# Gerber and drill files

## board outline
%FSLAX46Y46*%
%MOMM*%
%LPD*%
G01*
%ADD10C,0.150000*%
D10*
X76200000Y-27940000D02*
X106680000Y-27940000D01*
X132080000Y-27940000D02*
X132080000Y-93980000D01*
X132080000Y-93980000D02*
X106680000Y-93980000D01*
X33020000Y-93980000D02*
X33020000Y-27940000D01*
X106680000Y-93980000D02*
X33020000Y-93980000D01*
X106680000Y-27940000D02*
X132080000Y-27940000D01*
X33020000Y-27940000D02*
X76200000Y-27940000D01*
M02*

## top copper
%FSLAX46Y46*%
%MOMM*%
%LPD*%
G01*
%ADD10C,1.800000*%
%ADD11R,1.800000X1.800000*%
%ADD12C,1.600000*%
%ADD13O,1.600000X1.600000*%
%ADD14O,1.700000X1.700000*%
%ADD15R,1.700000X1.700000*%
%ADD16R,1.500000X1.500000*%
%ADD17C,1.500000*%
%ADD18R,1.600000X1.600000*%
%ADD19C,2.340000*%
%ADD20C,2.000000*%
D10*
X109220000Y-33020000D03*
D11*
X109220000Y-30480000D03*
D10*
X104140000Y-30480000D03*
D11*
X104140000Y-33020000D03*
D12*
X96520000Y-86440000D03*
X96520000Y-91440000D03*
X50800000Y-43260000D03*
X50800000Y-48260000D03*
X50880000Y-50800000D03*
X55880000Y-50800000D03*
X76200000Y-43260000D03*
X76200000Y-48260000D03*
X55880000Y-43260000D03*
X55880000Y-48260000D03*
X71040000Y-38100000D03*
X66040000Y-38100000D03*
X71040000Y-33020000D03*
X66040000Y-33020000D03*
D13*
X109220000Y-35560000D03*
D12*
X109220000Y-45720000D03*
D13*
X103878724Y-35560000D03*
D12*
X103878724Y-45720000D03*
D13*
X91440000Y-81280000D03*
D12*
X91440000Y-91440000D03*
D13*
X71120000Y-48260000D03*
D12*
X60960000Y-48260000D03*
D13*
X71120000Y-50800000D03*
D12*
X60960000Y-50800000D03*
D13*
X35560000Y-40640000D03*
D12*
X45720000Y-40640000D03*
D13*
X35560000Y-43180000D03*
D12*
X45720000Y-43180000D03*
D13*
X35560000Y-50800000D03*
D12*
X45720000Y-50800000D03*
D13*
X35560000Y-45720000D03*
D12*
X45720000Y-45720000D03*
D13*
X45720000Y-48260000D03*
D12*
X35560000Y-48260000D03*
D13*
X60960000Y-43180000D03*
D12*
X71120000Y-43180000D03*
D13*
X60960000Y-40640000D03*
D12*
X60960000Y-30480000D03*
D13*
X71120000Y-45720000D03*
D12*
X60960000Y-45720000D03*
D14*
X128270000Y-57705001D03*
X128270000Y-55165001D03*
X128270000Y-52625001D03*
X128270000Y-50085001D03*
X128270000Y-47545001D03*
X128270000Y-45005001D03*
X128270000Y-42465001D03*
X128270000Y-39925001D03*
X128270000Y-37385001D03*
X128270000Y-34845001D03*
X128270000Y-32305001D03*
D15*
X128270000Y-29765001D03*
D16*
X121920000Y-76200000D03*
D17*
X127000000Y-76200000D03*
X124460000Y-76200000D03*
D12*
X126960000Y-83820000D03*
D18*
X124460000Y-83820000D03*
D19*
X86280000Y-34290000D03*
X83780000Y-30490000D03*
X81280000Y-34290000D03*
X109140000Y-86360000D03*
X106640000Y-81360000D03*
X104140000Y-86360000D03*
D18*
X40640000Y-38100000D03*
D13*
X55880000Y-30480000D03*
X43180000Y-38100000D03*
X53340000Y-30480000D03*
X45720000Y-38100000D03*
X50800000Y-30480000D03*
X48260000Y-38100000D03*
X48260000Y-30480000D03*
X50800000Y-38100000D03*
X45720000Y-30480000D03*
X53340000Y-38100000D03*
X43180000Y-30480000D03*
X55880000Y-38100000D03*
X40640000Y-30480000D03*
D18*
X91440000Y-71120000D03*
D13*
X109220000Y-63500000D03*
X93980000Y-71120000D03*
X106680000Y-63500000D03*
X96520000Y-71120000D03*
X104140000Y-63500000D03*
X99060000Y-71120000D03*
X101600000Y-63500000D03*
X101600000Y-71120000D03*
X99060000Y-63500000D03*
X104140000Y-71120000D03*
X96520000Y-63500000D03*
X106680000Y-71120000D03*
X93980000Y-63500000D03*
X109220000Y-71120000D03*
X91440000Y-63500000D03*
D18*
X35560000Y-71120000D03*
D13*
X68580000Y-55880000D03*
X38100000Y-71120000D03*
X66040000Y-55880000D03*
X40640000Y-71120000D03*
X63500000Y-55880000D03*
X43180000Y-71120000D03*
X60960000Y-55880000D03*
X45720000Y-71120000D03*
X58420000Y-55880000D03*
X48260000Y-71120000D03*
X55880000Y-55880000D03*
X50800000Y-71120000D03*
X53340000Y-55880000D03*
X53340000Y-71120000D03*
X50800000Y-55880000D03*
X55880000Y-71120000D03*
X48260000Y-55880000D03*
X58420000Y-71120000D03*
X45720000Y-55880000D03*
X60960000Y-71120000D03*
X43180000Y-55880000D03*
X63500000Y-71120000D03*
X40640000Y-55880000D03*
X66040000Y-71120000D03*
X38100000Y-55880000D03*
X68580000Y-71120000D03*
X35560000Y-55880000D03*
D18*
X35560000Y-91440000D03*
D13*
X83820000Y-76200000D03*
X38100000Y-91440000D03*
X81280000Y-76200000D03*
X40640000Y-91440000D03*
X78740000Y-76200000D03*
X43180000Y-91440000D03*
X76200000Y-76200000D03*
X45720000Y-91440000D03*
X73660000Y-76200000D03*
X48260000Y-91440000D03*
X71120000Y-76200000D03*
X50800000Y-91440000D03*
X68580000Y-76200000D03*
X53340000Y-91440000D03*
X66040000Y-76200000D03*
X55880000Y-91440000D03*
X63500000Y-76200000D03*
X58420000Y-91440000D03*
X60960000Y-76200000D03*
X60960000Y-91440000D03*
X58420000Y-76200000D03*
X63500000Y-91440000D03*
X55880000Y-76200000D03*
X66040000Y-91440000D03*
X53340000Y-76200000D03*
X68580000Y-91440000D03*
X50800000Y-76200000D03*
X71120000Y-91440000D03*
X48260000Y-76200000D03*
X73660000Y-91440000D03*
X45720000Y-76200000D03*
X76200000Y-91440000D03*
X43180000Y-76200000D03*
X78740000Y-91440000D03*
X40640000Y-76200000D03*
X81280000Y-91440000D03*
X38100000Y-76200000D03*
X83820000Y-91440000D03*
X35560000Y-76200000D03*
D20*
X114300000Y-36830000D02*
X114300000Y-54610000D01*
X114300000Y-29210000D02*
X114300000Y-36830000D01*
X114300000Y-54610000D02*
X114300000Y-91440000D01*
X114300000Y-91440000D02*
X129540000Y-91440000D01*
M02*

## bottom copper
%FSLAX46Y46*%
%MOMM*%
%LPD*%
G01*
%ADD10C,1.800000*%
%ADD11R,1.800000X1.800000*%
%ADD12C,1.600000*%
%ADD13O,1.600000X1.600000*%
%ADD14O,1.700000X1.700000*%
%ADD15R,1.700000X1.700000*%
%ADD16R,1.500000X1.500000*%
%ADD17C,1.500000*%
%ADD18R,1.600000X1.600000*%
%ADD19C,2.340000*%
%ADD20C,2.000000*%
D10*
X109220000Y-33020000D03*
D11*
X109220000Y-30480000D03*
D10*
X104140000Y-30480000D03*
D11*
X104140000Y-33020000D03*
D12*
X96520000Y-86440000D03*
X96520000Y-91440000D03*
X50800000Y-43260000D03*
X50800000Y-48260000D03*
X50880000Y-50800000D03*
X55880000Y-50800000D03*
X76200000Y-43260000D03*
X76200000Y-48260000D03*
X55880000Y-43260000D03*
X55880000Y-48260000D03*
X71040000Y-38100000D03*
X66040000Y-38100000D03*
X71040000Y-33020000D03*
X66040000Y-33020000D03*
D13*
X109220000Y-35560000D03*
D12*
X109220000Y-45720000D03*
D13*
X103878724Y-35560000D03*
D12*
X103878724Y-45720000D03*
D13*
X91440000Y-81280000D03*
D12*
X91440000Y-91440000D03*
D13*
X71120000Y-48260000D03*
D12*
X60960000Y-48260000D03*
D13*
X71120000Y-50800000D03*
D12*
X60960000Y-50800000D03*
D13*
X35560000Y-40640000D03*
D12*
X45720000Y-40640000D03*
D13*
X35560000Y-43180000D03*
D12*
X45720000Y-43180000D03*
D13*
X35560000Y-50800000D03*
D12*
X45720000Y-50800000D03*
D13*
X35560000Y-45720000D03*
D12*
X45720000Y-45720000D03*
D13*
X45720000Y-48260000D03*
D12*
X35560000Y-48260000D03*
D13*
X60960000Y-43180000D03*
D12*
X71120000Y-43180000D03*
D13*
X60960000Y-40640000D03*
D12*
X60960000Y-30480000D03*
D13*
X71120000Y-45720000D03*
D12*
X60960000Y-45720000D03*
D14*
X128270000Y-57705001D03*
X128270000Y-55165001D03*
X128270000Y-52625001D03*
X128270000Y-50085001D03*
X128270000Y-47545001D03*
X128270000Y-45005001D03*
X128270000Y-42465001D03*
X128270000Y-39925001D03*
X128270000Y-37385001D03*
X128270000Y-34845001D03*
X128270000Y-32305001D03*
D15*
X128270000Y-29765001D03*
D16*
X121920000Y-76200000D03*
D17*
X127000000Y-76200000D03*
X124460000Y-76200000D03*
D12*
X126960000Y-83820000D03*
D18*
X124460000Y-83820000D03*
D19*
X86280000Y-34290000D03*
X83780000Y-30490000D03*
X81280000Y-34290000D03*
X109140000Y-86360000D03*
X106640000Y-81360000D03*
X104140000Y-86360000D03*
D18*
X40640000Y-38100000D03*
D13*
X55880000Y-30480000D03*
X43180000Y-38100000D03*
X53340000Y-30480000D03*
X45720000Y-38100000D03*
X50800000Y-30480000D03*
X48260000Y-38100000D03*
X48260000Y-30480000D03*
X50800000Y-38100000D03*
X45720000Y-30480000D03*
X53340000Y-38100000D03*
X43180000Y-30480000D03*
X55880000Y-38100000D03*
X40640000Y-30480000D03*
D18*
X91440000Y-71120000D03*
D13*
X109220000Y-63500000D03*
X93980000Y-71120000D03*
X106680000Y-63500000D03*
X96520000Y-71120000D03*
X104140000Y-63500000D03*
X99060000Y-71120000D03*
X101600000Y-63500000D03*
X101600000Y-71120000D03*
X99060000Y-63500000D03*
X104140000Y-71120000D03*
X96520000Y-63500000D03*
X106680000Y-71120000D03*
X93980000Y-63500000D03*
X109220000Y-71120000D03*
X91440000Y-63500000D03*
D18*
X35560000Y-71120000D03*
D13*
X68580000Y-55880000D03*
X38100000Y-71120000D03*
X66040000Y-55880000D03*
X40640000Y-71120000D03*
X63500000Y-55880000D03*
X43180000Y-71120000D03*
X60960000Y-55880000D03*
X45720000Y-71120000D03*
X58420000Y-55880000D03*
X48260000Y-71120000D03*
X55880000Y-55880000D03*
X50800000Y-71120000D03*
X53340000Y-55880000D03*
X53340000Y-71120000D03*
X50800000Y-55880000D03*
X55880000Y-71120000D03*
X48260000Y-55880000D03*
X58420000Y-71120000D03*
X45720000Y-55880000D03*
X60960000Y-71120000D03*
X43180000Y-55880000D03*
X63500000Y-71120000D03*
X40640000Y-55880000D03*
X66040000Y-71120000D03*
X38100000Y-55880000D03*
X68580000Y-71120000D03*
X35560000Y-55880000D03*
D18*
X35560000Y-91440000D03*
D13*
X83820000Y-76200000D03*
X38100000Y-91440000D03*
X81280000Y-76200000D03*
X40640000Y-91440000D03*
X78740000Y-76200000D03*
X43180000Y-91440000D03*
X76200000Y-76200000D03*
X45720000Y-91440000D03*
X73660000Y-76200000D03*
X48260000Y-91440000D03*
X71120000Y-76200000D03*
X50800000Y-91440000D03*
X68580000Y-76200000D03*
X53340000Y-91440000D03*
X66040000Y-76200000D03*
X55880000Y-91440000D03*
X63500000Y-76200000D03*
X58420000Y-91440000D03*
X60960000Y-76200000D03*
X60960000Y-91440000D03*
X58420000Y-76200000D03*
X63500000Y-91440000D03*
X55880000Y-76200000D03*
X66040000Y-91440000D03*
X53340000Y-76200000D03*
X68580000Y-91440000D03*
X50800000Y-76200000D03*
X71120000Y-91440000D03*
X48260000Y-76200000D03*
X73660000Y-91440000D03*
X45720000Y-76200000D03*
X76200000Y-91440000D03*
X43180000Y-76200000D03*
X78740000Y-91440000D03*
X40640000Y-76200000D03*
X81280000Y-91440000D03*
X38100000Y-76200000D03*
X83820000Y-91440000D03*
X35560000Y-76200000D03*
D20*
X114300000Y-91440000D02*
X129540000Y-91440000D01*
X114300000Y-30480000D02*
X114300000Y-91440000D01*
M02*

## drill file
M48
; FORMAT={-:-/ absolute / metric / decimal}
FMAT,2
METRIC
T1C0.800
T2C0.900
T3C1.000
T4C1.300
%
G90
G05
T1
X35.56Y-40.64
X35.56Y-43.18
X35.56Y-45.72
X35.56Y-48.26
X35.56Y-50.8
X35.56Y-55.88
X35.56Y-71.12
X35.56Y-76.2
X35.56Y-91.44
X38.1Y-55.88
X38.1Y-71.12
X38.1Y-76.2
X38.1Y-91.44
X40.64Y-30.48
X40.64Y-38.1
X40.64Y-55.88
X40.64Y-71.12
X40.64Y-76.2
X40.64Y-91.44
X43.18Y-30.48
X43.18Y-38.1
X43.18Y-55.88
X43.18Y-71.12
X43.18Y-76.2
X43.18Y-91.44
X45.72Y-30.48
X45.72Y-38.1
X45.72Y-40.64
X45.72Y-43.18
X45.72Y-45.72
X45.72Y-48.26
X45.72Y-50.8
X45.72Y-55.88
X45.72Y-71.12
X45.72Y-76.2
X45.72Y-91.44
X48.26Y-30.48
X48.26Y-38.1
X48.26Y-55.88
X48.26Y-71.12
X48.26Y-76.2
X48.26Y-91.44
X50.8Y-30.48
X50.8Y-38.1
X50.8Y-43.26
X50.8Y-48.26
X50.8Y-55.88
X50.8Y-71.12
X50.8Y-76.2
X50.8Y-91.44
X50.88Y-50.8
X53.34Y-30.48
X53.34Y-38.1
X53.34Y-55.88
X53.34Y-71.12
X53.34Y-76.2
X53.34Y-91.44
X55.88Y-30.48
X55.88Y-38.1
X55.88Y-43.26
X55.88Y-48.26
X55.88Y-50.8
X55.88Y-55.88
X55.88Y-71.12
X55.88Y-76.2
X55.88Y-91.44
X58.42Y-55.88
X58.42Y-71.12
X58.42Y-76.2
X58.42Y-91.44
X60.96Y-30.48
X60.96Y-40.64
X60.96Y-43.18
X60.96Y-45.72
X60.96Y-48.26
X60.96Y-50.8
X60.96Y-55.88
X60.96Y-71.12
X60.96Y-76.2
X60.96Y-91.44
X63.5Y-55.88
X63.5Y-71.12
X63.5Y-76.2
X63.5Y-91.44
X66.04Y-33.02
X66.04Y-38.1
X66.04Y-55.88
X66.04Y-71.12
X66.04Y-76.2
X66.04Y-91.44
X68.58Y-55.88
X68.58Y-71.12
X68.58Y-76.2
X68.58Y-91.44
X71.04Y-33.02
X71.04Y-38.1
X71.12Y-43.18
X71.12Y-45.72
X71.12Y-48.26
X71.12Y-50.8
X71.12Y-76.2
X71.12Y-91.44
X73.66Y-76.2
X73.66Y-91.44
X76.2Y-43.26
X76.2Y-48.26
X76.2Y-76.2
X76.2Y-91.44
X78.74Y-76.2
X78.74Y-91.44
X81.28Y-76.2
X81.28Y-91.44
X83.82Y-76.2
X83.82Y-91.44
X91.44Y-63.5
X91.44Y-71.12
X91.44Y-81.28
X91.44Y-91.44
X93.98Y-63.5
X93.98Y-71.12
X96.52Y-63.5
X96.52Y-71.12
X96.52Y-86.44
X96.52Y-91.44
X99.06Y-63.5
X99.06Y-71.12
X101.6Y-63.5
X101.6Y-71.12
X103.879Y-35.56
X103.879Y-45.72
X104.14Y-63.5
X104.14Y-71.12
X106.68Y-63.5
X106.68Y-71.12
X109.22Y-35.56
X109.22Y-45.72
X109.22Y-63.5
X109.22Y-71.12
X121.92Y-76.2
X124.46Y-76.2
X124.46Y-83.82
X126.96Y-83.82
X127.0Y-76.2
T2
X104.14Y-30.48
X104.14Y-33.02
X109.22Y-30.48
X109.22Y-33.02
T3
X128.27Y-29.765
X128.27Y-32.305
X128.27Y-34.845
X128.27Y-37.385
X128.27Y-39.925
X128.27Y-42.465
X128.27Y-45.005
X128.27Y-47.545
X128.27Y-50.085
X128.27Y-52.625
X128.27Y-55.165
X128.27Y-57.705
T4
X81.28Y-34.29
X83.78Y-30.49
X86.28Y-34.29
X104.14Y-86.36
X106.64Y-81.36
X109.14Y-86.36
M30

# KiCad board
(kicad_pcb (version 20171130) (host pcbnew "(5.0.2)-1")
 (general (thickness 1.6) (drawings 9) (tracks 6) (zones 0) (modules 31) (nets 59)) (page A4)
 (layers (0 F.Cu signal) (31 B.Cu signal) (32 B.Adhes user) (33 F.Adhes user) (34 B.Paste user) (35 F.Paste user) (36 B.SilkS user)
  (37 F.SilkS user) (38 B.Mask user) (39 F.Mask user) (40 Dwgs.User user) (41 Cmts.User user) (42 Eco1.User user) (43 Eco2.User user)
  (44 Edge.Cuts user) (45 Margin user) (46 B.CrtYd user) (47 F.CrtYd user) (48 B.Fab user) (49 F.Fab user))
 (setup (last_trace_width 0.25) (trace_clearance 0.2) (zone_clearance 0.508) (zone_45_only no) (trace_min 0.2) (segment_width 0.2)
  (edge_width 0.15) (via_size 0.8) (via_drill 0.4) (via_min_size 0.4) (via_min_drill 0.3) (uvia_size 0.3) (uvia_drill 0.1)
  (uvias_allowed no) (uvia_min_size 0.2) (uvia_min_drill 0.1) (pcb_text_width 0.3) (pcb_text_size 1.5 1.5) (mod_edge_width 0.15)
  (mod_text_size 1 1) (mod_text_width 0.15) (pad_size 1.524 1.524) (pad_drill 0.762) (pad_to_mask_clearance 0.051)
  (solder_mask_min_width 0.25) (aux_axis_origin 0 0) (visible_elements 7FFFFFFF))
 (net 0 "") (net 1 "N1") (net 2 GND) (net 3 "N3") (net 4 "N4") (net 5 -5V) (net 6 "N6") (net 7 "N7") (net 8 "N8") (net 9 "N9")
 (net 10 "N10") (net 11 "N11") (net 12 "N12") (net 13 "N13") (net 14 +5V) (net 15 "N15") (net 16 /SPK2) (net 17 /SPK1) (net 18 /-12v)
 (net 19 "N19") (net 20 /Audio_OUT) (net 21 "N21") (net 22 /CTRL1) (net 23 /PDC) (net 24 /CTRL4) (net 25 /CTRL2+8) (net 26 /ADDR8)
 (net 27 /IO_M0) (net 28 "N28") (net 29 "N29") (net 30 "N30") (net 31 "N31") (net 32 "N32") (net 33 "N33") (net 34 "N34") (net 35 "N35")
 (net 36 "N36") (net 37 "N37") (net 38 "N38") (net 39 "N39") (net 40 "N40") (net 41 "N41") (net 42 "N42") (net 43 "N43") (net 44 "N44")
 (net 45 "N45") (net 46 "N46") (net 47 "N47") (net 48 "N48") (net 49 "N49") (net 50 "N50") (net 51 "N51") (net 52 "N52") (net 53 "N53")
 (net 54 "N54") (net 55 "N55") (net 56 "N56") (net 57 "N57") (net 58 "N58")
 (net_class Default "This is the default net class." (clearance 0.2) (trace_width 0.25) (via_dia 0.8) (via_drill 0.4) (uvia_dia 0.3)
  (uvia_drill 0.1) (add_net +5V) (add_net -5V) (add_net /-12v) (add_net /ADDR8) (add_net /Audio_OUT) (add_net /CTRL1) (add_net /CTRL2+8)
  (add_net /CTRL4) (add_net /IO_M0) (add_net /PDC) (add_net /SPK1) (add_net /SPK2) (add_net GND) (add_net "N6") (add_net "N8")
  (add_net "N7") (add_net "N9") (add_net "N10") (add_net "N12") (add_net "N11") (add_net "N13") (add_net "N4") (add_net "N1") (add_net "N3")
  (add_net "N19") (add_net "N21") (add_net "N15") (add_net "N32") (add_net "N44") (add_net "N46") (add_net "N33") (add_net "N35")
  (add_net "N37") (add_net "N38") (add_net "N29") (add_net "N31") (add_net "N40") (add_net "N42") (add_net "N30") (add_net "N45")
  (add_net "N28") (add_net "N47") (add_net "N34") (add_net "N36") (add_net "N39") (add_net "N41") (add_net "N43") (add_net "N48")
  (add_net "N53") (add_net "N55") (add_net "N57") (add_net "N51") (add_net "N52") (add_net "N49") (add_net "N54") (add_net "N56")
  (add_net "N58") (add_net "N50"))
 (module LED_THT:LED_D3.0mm (layer F.Cu) (at 109.22 30.48 270)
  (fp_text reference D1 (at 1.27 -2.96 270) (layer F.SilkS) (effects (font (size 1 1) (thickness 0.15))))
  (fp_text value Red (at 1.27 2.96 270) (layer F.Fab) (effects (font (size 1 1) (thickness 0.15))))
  (pad 2 thru_hole circle (at 2.54 0 270) (size 1.8 1.8) (drill 0.9) (layers *.Cu *.Mask) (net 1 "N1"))
  (pad 1 thru_hole rect (at 0 0 270) (size 1.8 1.8) (drill 0.9) (layers *.Cu *.Mask) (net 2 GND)))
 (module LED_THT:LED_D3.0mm (layer F.Cu) (at 104.14 33.02 90)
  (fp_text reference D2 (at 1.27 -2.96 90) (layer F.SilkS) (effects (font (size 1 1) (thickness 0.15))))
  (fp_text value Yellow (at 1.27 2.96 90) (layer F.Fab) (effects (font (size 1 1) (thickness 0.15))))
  (pad 2 thru_hole circle (at 2.54 0 90) (size 1.8 1.8) (drill 0.9) (layers *.Cu *.Mask) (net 2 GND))
  (pad 1 thru_hole rect (at 0 0 90) (size 1.8 1.8) (drill 0.9) (layers *.Cu *.Mask) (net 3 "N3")))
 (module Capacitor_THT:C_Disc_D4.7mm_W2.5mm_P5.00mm (layer F.Cu) (at 96.52 91.44 90)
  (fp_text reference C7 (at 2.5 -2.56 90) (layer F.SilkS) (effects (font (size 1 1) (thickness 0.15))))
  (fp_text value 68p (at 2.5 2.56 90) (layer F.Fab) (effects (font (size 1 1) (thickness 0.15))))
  (pad 2 thru_hole circle (at 5 0 90) (size 1.6 1.6) (drill 0.8) (layers *.Cu *.Mask) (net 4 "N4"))
  (pad 1 thru_hole circle (at 0 0 90) (size 1.6 1.6) (drill 0.8) (layers *.Cu *.Mask) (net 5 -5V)))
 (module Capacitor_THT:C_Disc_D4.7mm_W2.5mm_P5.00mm (layer F.Cu) (at 50.8 48.26 90)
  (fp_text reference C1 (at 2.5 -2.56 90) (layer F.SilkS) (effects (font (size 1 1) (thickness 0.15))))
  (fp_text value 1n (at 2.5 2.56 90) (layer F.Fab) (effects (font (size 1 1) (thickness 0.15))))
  (pad 2 thru_hole circle (at 5 0 90) (size 1.6 1.6) (drill 0.8) (layers *.Cu *.Mask) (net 2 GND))
  (pad 1 thru_hole circle (at 0 0 90) (size 1.6 1.6) (drill 0.8) (layers *.Cu *.Mask) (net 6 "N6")))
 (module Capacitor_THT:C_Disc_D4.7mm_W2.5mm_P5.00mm (layer F.Cu) (at 55.88 50.8 180)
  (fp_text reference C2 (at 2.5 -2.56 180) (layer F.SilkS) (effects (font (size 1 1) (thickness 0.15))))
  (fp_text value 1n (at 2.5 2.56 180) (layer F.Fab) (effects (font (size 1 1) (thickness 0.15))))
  (pad 2 thru_hole circle (at 5 0 180) (size 1.6 1.6) (drill 0.8) (layers *.Cu *.Mask) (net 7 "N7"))
  (pad 1 thru_hole circle (at 0 0 180) (size 1.6 1.6) (drill 0.8) (layers *.Cu *.Mask) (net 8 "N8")))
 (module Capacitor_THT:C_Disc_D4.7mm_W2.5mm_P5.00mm (layer F.Cu) (at 76.2 48.26 90)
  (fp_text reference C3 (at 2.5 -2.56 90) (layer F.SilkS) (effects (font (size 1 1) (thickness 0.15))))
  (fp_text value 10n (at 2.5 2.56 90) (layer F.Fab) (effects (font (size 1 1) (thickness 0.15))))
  (pad 2 thru_hole circle (at 5 0 90) (size 1.6 1.6) (drill 0.8) (layers *.Cu *.Mask) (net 2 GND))
  (pad 1 thru_hole circle (at 0 0 90) (size 1.6 1.6) (drill 0.8) (layers *.Cu *.Mask) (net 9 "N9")))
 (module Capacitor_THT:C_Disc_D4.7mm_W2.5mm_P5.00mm (layer F.Cu) (at 55.88 48.26 90)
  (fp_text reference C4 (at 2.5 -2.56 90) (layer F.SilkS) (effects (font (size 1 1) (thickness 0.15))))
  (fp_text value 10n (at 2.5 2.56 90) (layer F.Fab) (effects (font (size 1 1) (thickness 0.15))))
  (pad 2 thru_hole circle (at 5 0 90) (size 1.6 1.6) (drill 0.8) (layers *.Cu *.Mask) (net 2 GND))
  (pad 1 thru_hole circle (at 0 0 90) (size 1.6 1.6) (drill 0.8) (layers *.Cu *.Mask) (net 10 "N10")))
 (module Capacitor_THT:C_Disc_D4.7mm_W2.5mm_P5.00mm (layer F.Cu) (at 66.04 38.1)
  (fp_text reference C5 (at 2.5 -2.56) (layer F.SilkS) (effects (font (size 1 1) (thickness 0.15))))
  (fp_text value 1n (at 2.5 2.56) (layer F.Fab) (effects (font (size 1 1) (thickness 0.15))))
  (pad 2 thru_hole circle (at 5 0) (size 1.6 1.6) (drill 0.8) (layers *.Cu *.Mask) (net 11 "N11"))
  (pad 1 thru_hole circle (at 0 0) (size 1.6 1.6) (drill 0.8) (layers *.Cu *.Mask) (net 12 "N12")))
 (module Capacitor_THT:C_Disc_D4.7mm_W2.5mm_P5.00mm (layer F.Cu) (at 66.04 33.02)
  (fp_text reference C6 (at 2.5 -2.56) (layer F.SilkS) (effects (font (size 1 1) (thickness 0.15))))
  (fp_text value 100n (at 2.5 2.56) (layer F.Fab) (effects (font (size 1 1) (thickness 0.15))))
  (pad 2 thru_hole circle (at 5 0) (size 1.6 1.6) (drill 0.8) (layers *.Cu *.Mask) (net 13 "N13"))
  (pad 1 thru_hole circle (at 0 0) (size 1.6 1.6) (drill 0.8) (layers *.Cu *.Mask) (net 12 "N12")))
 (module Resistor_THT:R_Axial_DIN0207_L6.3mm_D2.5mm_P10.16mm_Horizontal (layer F.Cu) (at 109.22 45.72 90)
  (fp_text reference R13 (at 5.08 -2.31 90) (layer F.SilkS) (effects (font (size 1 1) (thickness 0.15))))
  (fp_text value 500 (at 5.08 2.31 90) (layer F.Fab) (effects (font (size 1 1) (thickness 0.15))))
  (pad 2 thru_hole oval (at 10.16 0 90) (size 1.6 1.6) (drill 0.8) (layers *.Cu *.Mask) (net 1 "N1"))
  (pad 1 thru_hole circle (at 0 0 90) (size 1.6 1.6) (drill 0.8) (layers *.Cu *.Mask) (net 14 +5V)))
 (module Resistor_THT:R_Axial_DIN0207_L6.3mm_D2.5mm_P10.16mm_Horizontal (layer F.Cu) (at 103.878724 45.72 90)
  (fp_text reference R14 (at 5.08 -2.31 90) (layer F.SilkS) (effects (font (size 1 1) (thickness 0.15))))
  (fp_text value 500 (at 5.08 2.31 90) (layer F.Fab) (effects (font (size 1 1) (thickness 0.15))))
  (pad 2 thru_hole oval (at 10.16 0 90) (size 1.6 1.6) (drill 0.8) (layers *.Cu *.Mask) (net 3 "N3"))
  (pad 1 thru_hole circle (at 0 0 90) (size 1.6 1.6) (drill 0.8) (layers *.Cu *.Mask) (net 5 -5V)))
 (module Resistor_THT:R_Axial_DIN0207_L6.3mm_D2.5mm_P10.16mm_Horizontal (layer F.Cu) (at 91.44 91.44 90)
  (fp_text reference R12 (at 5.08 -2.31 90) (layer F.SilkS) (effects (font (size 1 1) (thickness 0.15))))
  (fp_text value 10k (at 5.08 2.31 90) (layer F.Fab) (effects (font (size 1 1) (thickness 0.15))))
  (pad 2 thru_hole oval (at 10.16 0 90) (size 1.6 1.6) (drill 0.8) (layers *.Cu *.Mask) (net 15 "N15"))
  (pad 1 thru_hole circle (at 0 0 90) (size 1.6 1.6) (drill 0.8) (layers *.Cu *.Mask) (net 5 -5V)))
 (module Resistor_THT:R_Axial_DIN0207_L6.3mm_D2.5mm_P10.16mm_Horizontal (layer F.Cu) (at 60.96 48.26)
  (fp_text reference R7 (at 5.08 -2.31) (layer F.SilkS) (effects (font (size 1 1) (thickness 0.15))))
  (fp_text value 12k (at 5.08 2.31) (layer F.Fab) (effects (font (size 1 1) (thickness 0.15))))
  (pad 2 thru_hole oval (at 10.16 0) (size 1.6 1.6) (drill 0.8) (layers *.Cu *.Mask) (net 9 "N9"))
  (pad 1 thru_hole circle (at 0 0) (size 1.6 1.6) (drill 0.8) (layers *.Cu *.Mask) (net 8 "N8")))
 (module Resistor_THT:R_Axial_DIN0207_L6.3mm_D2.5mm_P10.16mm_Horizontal (layer F.Cu) (at 60.96 50.8)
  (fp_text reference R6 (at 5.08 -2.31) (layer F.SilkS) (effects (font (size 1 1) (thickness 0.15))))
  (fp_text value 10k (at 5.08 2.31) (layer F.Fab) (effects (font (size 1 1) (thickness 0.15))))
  (pad 2 thru_hole oval (at 10.16 0) (size 1.6 1.6) (drill 0.8) (layers *.Cu *.Mask) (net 7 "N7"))
  (pad 1 thru_hole circle (at 0 0) (size 1.6 1.6) (drill 0.8) (layers *.Cu *.Mask) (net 8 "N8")))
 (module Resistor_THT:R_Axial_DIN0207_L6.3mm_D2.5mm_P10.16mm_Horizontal (layer F.Cu) (at 45.72 40.64 180)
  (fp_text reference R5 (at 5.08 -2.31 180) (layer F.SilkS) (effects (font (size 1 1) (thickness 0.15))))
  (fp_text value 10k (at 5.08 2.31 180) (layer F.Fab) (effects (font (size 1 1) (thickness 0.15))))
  (pad 2 thru_hole oval (at 10.16 0 180) (size 1.6 1.6) (drill 0.8) (layers *.Cu *.Mask) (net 2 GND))
  (pad 1 thru_hole circle (at 0 0 180) (size 1.6 1.6) (drill 0.8) (layers *.Cu *.Mask) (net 6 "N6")))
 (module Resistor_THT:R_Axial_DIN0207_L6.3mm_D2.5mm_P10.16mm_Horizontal (layer F.Cu) (at 45.72 43.18 180)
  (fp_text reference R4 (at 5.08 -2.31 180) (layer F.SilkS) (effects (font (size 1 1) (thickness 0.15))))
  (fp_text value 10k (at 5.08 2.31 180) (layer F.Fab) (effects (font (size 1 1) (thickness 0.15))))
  (pad 2 thru_hole oval (at 10.16 0 180) (size 1.6 1.6) (drill 0.8) (layers *.Cu *.Mask) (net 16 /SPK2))
  (pad 1 thru_hole circle (at 0 0 180) (size 1.6 1.6) (drill 0.8) (layers *.Cu *.Mask) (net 6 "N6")))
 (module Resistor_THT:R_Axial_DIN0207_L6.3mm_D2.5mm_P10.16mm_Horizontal (layer F.Cu) (at 45.72 50.8 180)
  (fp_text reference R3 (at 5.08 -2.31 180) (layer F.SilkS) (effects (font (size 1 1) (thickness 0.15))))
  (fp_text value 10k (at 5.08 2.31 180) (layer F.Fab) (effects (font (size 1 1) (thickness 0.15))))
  (pad 2 thru_hole oval (at 10.16 0 180) (size 1.6 1.6) (drill 0.8) (layers *.Cu *.Mask) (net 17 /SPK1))
  (pad 1 thru_hole circle (at 0 0 180) (size 1.6 1.6) (drill 0.8) (layers *.Cu *.Mask) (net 7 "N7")))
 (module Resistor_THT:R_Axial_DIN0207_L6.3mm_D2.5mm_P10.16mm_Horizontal (layer F.Cu) (at 45.72 45.72 180)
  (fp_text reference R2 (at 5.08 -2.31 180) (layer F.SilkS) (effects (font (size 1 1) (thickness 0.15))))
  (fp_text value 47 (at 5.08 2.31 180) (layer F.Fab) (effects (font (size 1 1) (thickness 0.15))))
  (pad 2 thru_hole oval (at 10.16 0 180) (size 1.6 1.6) (drill 0.8) (layers *.Cu *.Mask) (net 16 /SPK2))
  (pad 1 thru_hole circle (at 0 0 180) (size 1.6 1.6) (drill 0.8) (layers *.Cu *.Mask) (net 5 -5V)))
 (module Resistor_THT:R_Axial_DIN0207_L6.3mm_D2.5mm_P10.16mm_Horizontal (layer F.Cu) (at 35.56 48.26)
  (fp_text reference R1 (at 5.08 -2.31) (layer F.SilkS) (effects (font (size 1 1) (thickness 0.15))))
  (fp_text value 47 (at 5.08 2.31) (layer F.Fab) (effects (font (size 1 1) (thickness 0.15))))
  (pad 2 thru_hole oval (at 10.16 0) (size 1.6 1.6) (drill 0.8) (layers *.Cu *.Mask) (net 5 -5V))
  (pad 1 thru_hole circle (at 0 0) (size 1.6 1.6) (drill 0.8) (layers *.Cu *.Mask) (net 17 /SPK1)))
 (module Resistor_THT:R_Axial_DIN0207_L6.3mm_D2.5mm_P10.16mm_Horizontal (layer F.Cu) (at 71.12 43.18 180)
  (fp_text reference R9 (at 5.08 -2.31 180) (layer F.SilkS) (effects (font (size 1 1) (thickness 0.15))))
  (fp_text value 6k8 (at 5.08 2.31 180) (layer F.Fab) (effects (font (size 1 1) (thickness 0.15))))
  (pad 2 thru_hole oval (at 10.16 0 180) (size 1.6 1.6) (drill 0.8) (layers *.Cu *.Mask) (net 10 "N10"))
  (pad 1 thru_hole circle (at 0 0 180) (size 1.6 1.6) (drill 0.8) (layers *.Cu *.Mask) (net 11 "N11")))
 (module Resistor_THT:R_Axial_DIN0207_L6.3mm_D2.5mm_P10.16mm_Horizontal (layer F.Cu) (at 60.96 30.48 270)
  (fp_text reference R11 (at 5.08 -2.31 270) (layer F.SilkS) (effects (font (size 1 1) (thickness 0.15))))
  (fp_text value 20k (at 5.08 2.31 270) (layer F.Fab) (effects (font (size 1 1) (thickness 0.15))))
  (pad 2 thru_hole oval (at 10.16 0 270) (size 1.6 1.6) (drill 0.8) (layers *.Cu *.Mask) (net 10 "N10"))
  (pad 1 thru_hole circle (at 0 0 270) (size 1.6 1.6) (drill 0.8) (layers *.Cu *.Mask) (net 12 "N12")))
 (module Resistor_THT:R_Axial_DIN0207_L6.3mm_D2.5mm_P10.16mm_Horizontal (layer F.Cu) (at 60.96 45.72)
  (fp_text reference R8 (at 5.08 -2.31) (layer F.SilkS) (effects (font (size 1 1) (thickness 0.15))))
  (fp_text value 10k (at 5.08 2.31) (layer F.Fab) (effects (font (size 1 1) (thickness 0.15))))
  (pad 2 thru_hole oval (at 10.16 0) (size 1.6 1.6) (drill 0.8) (layers *.Cu *.Mask) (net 9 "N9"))
  (pad 1 thru_hole circle (at 0 0) (size 1.6 1.6) (drill 0.8) (layers *.Cu *.Mask) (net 10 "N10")))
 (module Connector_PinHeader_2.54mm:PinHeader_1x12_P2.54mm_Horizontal (layer F.Cu) (at 128.27 29.765001)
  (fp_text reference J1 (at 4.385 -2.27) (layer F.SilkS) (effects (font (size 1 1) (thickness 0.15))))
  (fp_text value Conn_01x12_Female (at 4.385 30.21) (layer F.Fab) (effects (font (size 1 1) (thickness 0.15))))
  (pad 12 thru_hole oval (at 0 27.94) (size 1.7 1.7) (drill 1) (layers *.Cu *.Mask) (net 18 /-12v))
  (pad 11 thru_hole oval (at 0 25.4) (size 1.7 1.7) (drill 1) (layers *.Cu *.Mask) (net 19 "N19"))
  (pad 10 thru_hole oval (at 0 22.86) (size 1.7 1.7) (drill 1) (layers *.Cu *.Mask) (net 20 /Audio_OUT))
  (pad 9 thru_hole oval (at 0 20.32) (size 1.7 1.7) (drill 1) (layers *.Cu *.Mask) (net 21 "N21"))
  (pad 8 thru_hole oval (at 0 17.78) (size 1.7 1.7) (drill 1) (layers *.Cu *.Mask) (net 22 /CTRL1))
  (pad 7 thru_hole oval (at 0 15.24) (size 1.7 1.7) (drill 1) (layers *.Cu *.Mask) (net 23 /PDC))
  (pad 6 thru_hole oval (at 0 12.7) (size 1.7 1.7) (drill 1) (layers *.Cu *.Mask) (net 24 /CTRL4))
  (pad 5 thru_hole oval (at 0 10.16) (size 1.7 1.7) (drill 1) (layers *.Cu *.Mask) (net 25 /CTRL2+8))
  (pad 4 thru_hole oval (at 0 7.62) (size 1.7 1.7) (drill 1) (layers *.Cu *.Mask) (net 14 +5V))
  (pad 3 thru_hole oval (at 0 5.08) (size 1.7 1.7) (drill 1) (layers *.Cu *.Mask) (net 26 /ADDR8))
  (pad 2 thru_hole oval (at 0 2.54) (size 1.7 1.7) (drill 1) (layers *.Cu *.Mask) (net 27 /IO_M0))
  (pad 1 thru_hole rect (at 0 0) (size 1.7 1.7) (drill 1) (layers *.Cu *.Mask) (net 2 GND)))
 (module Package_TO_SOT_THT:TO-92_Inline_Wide (layer F.Cu) (at 121.92 76.2)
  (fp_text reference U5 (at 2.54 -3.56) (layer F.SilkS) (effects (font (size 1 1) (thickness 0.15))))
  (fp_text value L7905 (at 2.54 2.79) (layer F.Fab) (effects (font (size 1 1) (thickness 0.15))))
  (pad 1 thru_hole rect (at 0 0 90) (size 1.5 1.5) (drill 0.8) (layers *.Cu *.Mask) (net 2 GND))
  (pad 3 thru_hole circle (at 5.08 0 90) (size 1.5 1.5) (drill 0.8) (layers *.Cu *.Mask) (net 5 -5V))
  (pad 2 thru_hole circle (at 2.54 0 90) (size 1.5 1.5) (drill 0.8) (layers *.Cu *.Mask) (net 18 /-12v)))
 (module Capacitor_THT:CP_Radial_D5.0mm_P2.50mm (layer F.Cu) (at 124.46 83.82)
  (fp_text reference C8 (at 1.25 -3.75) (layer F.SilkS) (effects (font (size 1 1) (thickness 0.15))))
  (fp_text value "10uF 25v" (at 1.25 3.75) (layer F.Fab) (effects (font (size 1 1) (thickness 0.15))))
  (pad 2 thru_hole circle (at 2.5 0) (size 1.6 1.6) (drill 0.8) (layers *.Cu *.Mask) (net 5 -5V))
  (pad 1 thru_hole rect (at 0 0) (size 1.6 1.6) (drill 0.8) (layers *.Cu *.Mask) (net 2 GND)))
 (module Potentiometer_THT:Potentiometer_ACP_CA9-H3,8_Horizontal (layer F.Cu) (at 81.28 34.29 90)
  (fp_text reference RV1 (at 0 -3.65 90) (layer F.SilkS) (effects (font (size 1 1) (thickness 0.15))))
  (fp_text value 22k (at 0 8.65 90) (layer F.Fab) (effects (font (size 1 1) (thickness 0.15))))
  (pad 3 thru_hole circle (at 0 5 90) (size 2.34 2.34) (drill 1.3) (layers *.Cu *.Mask) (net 2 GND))
  (pad 2 thru_hole circle (at 3.8 2.5 90) (size 2.34 2.34) (drill 1.3) (layers *.Cu *.Mask) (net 20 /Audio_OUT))
  (pad 1 thru_hole circle (at 0 0 90) (size 2.34 2.34) (drill 1.3) (layers *.Cu *.Mask) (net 13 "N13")))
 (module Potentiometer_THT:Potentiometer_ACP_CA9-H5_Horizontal (layer F.Cu) (at 104.14 86.36 90)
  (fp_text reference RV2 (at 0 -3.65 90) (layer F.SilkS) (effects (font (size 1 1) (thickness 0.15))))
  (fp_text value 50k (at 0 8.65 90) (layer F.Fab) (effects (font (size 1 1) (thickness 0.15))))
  (pad 3 thru_hole circle (at 0 5 90) (size 2.34 2.34) (drill 1.3) (layers *.Cu *.Mask) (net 4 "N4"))
  (pad 2 thru_hole circle (at 5 2.5 90) (size 2.34 2.34) (drill 1.3) (layers *.Cu *.Mask) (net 4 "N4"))
  (pad 1 thru_hole circle (at 0 0 90) (size 2.34 2.34) (drill 1.3) (layers *.Cu *.Mask) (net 15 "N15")))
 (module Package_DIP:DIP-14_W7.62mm (layer F.Cu) (at 40.64 38.1 90)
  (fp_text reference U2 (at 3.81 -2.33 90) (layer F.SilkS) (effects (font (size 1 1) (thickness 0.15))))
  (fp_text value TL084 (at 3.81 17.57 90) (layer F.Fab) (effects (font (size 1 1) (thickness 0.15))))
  (pad 1 thru_hole rect (at 0 0 90) (size 1.6 1.6) (drill 0.8) (layers *.Cu *.Mask) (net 8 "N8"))
  (pad 8 thru_hole oval (at 7.62 15.24 90) (size 1.6 1.6) (drill 0.8) (layers *.Cu *.Mask))
  (pad 2 thru_hole oval (at 0 2.54 90) (size 1.6 1.6) (drill 0.8) (layers *.Cu *.Mask) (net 7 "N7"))
  (pad 9 thru_hole oval (at 7.62 12.7 90) (size 1.6 1.6) (drill 0.8) (layers *.Cu *.Mask))
  (pad 3 thru_hole oval (at 0 5.08 90) (size 1.6 1.6) (drill 0.8) (layers *.Cu *.Mask) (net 6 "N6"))
  (pad 10 thru_hole oval (at 7.62 10.16 90) (size 1.6 1.6) (drill 0.8) (layers *.Cu *.Mask))
  (pad 4 thru_hole oval (at 0 7.62 90) (size 1.6 1.6) (drill 0.8) (layers *.Cu *.Mask) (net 14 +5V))
  (pad 11 thru_hole oval (at 7.62 7.62 90) (size 1.6 1.6) (drill 0.8) (layers *.Cu *.Mask) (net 5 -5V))
  (pad 5 thru_hole oval (at 0 10.16 90) (size 1.6 1.6) (drill 0.8) (layers *.Cu *.Mask) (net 2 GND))
  (pad 12 thru_hole oval (at 7.62 5.08 90) (size 1.6 1.6) (drill 0.8) (layers *.Cu *.Mask))
  (pad 6 thru_hole oval (at 0 12.7 90) (size 1.6 1.6) (drill 0.8) (layers *.Cu *.Mask) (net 11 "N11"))
  (pad 13 thru_hole oval (at 7.62 2.54 90) (size 1.6 1.6) (drill 0.8) (layers *.Cu *.Mask))
  (pad 7 thru_hole oval (at 0 15.24 90) (size 1.6 1.6) (drill 0.8) (layers *.Cu *.Mask) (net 12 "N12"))
  (pad 14 thru_hole oval (at 7.62 0 90) (size 1.6 1.6) (drill 0.8) (layers *.Cu *.Mask)))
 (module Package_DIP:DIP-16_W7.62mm (layer F.Cu) (at 91.44 71.12 90)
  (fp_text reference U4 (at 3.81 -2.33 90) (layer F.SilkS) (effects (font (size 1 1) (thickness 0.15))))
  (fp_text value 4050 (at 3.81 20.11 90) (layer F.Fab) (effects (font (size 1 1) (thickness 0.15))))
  (pad 1 thru_hole rect (at 0 0 90) (size 1.6 1.6) (drill 0.8) (layers *.Cu *.Mask) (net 14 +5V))
  (pad 9 thru_hole oval (at 7.62 17.78 90) (size 1.6 1.6) (drill 0.8) (layers *.Cu *.Mask) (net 23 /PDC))
  (pad 2 thru_hole oval (at 0 2.54 90) (size 1.6 1.6) (drill 0.8) (layers *.Cu *.Mask) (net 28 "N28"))
  (pad 10 thru_hole oval (at 7.62 15.24 90) (size 1.6 1.6) (drill 0.8) (layers *.Cu *.Mask) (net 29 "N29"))
  (pad 3 thru_hole oval (at 0 5.08 90) (size 1.6 1.6) (drill 0.8) (layers *.Cu *.Mask) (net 26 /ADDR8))
  (pad 11 thru_hole oval (at 7.62 12.7 90) (size 1.6 1.6) (drill 0.8) (layers *.Cu *.Mask))
  (pad 4 thru_hole oval (at 0 7.62 90) (size 1.6 1.6) (drill 0.8) (layers *.Cu *.Mask) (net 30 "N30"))
  (pad 12 thru_hole oval (at 7.62 10.16 90) (size 1.6 1.6) (drill 0.8) (layers *.Cu *.Mask))
  (pad 5 thru_hole oval (at 0 10.16 90) (size 1.6 1.6) (drill 0.8) (layers *.Cu *.Mask) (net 25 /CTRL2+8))
  (pad 13 thru_hole oval (at 7.62 7.62 90) (size 1.6 1.6) (drill 0.8) (layers *.Cu *.Mask))
  (pad 6 thru_hole oval (at 0 12.7 90) (size 1.6 1.6) (drill 0.8) (layers *.Cu *.Mask) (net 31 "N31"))
  (pad 14 thru_hole oval (at 7.62 5.08 90) (size 1.6 1.6) (drill 0.8) (layers *.Cu *.Mask))
  (pad 7 thru_hole oval (at 0 15.24 90) (size 1.6 1.6) (drill 0.8) (layers *.Cu *.Mask) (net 24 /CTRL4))
  (pad 15 thru_hole oval (at 7.62 2.54 90) (size 1.6 1.6) (drill 0.8) (layers *.Cu *.Mask))
  (pad 8 thru_hole oval (at 0 17.78 90) (size 1.6 1.6) (drill 0.8) (layers *.Cu *.Mask) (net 2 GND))
  (pad 16 thru_hole oval (at 7.62 0 90) (size 1.6 1.6) (drill 0.8) (layers *.Cu *.Mask)))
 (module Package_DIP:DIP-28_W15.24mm (layer F.Cu) (at 35.56 71.12 90)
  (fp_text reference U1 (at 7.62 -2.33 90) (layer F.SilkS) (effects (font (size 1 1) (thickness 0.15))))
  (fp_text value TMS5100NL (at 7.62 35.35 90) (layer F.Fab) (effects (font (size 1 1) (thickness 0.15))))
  (pad 1 thru_hole rect (at 0 0 90) (size 1.6 1.6) (drill 0.8) (layers *.Cu *.Mask) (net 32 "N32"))
  (pad 15 thru_hole oval (at 15.24 33.02 90) (size 1.6 1.6) (drill 0.8) (layers *.Cu *.Mask) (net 27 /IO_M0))
  (pad 2 thru_hole oval (at 0 2.54 90) (size 1.6 1.6) (drill 0.8) (layers *.Cu *.Mask) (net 29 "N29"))
  (pad 16 thru_hole oval (at 15.24 30.48 90) (size 1.6 1.6) (drill 0.8) (layers *.Cu *.Mask) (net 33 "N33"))
  (pad 3 thru_hole oval (at 0 5.08 90) (size 1.6 1.6) (drill 0.8) (layers *.Cu *.Mask) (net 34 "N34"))
  (pad 17 thru_hole oval (at 15.24 27.94 90) (size 1.6 1.6) (drill 0.8) (layers *.Cu *.Mask) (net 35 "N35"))
  (pad 4 thru_hole oval (at 0 7.62 90) (size 1.6 1.6) (drill 0.8) (layers *.Cu *.Mask) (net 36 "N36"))
  (pad 18 thru_hole oval (at 15.24 25.4 90) (size 1.6 1.6) (drill 0.8) (layers *.Cu *.Mask) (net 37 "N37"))
  (pad 5 thru_hole oval (at 0 10.16 90) (size 1.6 1.6) (drill 0.8) (layers *.Cu *.Mask) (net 5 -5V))
  (pad 19 thru_hole oval (at 15.24 22.86 90) (size 1.6 1.6) (drill 0.8) (layers *.Cu *.Mask) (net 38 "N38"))
  (pad 6 thru_hole oval (at 0 12.7 90) (size 1.6 1.6) (drill 0.8) (layers *.Cu *.Mask) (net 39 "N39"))
  (pad 20 thru_hole oval (at 15.24 20.32 90) (size 1.6 1.6) (drill 0.8) (layers *.Cu *.Mask) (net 31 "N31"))
  (pad 7 thru_hole oval (at 0 15.24 90) (size 1.6 1.6) (drill 0.8) (layers *.Cu *.Mask) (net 4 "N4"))
  (pad 21 thru_hole oval (at 15.24 17.78 90) (size 1.6 1.6) (drill 0.8) (layers *.Cu *.Mask) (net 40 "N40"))
  (pad 8 thru_hole oval (at 0 17.78 90) (size 1.6 1.6) (drill 0.8) (layers *.Cu *.Mask) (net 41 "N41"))
  (pad 22 thru_hole oval (at 15.24 15.24 90) (size 1.6 1.6) (drill 0.8) (layers *.Cu *.Mask) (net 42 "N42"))
  (pad 9 thru_hole oval (at 0 20.32 90) (size 1.6 1.6) (drill 0.8) (layers *.Cu *.Mask) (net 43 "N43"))
  (pad 23 thru_hole oval (at 15.24 12.7 90) (size 1.6 1.6) (drill 0.8) (layers *.Cu *.Mask) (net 30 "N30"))
  (pad 10 thru_hole oval (at 0 22.86 90) (size 1.6 1.6) (drill 0.8) (layers *.Cu *.Mask) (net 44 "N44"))
  (pad 24 thru_hole oval (at 15.24 10.16 90) (size 1.6 1.6) (drill 0.8) (layers *.Cu *.Mask) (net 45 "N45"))
  (pad 11 thru_hole oval (at 0 25.4 90) (size 1.6 1.6) (drill 0.8) (layers *.Cu *.Mask) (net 17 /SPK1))
  (pad 25 thru_hole oval (at 15.24 7.62 90) (size 1.6 1.6) (drill 0.8) (layers *.Cu *.Mask) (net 22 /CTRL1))
  (pad 12 thru_hole oval (at 0 27.94 90) (size 1.6 1.6) (drill 0.8) (layers *.Cu *.Mask) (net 16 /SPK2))
  (pad 26 thru_hole oval (at 15.24 5.08 90) (size 1.6 1.6) (drill 0.8) (layers *.Cu *.Mask) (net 28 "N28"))
  (pad 13 thru_hole oval (at 0 30.48 90) (size 1.6 1.6) (drill 0.8) (layers *.Cu *.Mask) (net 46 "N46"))
  (pad 27 thru_hole oval (at 15.24 2.54 90) (size 1.6 1.6) (drill 0.8) (layers *.Cu *.Mask) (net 30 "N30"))
  (pad 14 thru_hole oval (at 0 33.02 90) (size 1.6 1.6) (drill 0.8) (layers *.Cu *.Mask) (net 14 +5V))
  (pad 28 thru_hole oval (at 15.24 0 90) (size 1.6 1.6) (drill 0.8) (layers *.Cu *.Mask) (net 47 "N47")))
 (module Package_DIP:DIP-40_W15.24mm (layer F.Cu) (at 35.56 91.44 90)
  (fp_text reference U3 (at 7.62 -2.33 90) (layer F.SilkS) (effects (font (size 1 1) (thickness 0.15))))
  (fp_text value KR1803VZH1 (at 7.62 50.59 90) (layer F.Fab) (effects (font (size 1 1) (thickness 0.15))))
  (pad 1 thru_hole rect (at 0 0 90) (size 1.6 1.6) (drill 0.8) (layers *.Cu *.Mask) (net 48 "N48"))
  (pad 21 thru_hole oval (at 15.24 48.26 90) (size 1.6 1.6) (drill 0.8) (layers *.Cu *.Mask))
  (pad 2 thru_hole oval (at 0 2.54 90) (size 1.6 1.6) (drill 0.8) (layers *.Cu *.Mask) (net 29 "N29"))
  (pad 22 thru_hole oval (at 15.24 45.72 90) (size 1.6 1.6) (drill 0.8) (layers *.Cu *.Mask) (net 27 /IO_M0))
  (pad 3 thru_hole oval (at 0 5.08 90) (size 1.6 1.6) (drill 0.8) (layers *.Cu *.Mask) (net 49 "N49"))
  (pad 23 thru_hole oval (at 15.24 43.18 90) (size 1.6 1.6) (drill 0.8) (layers *.Cu *.Mask))
  (pad 4 thru_hole oval (at 0 7.62 90) (size 1.6 1.6) (drill 0.8) (layers *.Cu *.Mask) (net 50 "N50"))
  (pad 24 thru_hole oval (at 15.24 40.64 90) (size 1.6 1.6) (drill 0.8) (layers *.Cu *.Mask))
  (pad 5 thru_hole oval (at 0 10.16 90) (size 1.6 1.6) (drill 0.8) (layers *.Cu *.Mask) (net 5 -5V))
  (pad 25 thru_hole oval (at 15.24 38.1 90) (size 1.6 1.6) (drill 0.8) (layers *.Cu *.Mask))
  (pad 6 thru_hole oval (at 0 12.7 90) (size 1.6 1.6) (drill 0.8) (layers *.Cu *.Mask))
  (pad 26 thru_hole oval (at 15.24 35.56 90) (size 1.6 1.6) (drill 0.8) (layers *.Cu *.Mask))
  (pad 7 thru_hole oval (at 0 15.24 90) (size 1.6 1.6) (drill 0.8) (layers *.Cu *.Mask))
  (pad 27 thru_hole oval (at 15.24 33.02 90) (size 1.6 1.6) (drill 0.8) (layers *.Cu *.Mask) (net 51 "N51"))
  (pad 8 thru_hole oval (at 0 17.78 90) (size 1.6 1.6) (drill 0.8) (layers *.Cu *.Mask))
  (pad 28 thru_hole oval (at 15.24 30.48 90) (size 1.6 1.6) (drill 0.8) (layers *.Cu *.Mask) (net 31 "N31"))
  (pad 9 thru_hole oval (at 0 20.32 90) (size 1.6 1.6) (drill 0.8) (layers *.Cu *.Mask))
  (pad 29 thru_hole oval (at 15.24 27.94 90) (size 1.6 1.6) (drill 0.8) (layers *.Cu *.Mask) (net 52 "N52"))
  (pad 10 thru_hole oval (at 0 22.86 90) (size 1.6 1.6) (drill 0.8) (layers *.Cu *.Mask))
  (pad 30 thru_hole oval (at 15.24 25.4 90) (size 1.6 1.6) (drill 0.8) (layers *.Cu *.Mask))
  (pad 11 thru_hole oval (at 0 25.4 90) (size 1.6 1.6) (drill 0.8) (layers *.Cu *.Mask) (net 4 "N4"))
  (pad 31 thru_hole oval (at 15.24 22.86 90) (size 1.6 1.6) (drill 0.8) (layers *.Cu *.Mask))
  (pad 12 thru_hole oval (at 0 27.94 90) (size 1.6 1.6) (drill 0.8) (layers *.Cu *.Mask) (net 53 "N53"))
  (pad 32 thru_hole oval (at 15.24 20.32 90) (size 1.6 1.6) (drill 0.8) (layers *.Cu *.Mask) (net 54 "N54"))
  (pad 13 thru_hole oval (at 0 30.48 90) (size 1.6 1.6) (drill 0.8) (layers *.Cu *.Mask) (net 5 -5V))
  (pad 33 thru_hole oval (at 15.24 17.78 90) (size 1.6 1.6) (drill 0.8) (layers *.Cu *.Mask) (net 30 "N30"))
  (pad 14 thru_hole oval (at 0 33.02 90) (size 1.6 1.6) (drill 0.8) (layers *.Cu *.Mask) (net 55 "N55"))
  (pad 34 thru_hole oval (at 15.24 15.24 90) (size 1.6 1.6) (drill 0.8) (layers *.Cu *.Mask) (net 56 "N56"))
  (pad 15 thru_hole oval (at 0 35.56 90) (size 1.6 1.6) (drill 0.8) (layers *.Cu *.Mask) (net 17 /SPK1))
  (pad 35 thru_hole oval (at 15.24 12.7 90) (size 1.6 1.6) (drill 0.8) (layers *.Cu *.Mask))
  (pad 16 thru_hole oval (at 0 38.1 90) (size 1.6 1.6) (drill 0.8) (layers *.Cu *.Mask) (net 16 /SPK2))
  (pad 36 thru_hole oval (at 15.24 10.16 90) (size 1.6 1.6) (drill 0.8) (layers *.Cu *.Mask) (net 22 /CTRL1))
  (pad 17 thru_hole oval (at 0 40.64 90) (size 1.6 1.6) (drill 0.8) (layers *.Cu *.Mask) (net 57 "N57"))
  (pad 37 thru_hole oval (at 15.24 7.62 90) (size 1.6 1.6) (drill 0.8) (layers *.Cu *.Mask) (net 28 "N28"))
  (pad 18 thru_hole oval (at 0 43.18 90) (size 1.6 1.6) (drill 0.8) (layers *.Cu *.Mask) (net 14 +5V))
  (pad 38 thru_hole oval (at 15.24 5.08 90) (size 1.6 1.6) (drill 0.8) (layers *.Cu *.Mask) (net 30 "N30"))
  (pad 19 thru_hole oval (at 0 45.72 90) (size 1.6 1.6) (drill 0.8) (layers *.Cu *.Mask))
  (pad 39 thru_hole oval (at 15.24 2.54 90) (size 1.6 1.6) (drill 0.8) (layers *.Cu *.Mask) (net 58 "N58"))
  (pad 20 thru_hole oval (at 0 48.26 90) (size 1.6 1.6) (drill 0.8) (layers *.Cu *.Mask))
  (pad 40 thru_hole oval (at 15.24 0 90) (size 1.6 1.6) (drill 0.8) (layers *.Cu *.Mask) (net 14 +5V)))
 (gr_line (start 76.2 27.94) (end 106.68 27.94) (layer Edge.Cuts) (width 0.15))
 (gr_line (start 132.08 27.94) (end 132.08 93.98) (layer Edge.Cuts) (width 0.15))
 (gr_line (start 132.08 93.98) (end 106.68 93.98) (layer Edge.Cuts) (width 0.15))
 (gr_line (start 33.02 93.98) (end 33.02 27.94) (layer Edge.Cuts) (width 0.15))
 (gr_line (start 106.68 93.98) (end 33.02 93.98) (layer Edge.Cuts) (width 0.15))
 (gr_line (start 106.68 27.94) (end 132.08 27.94) (layer Edge.Cuts) (width 0.15))
 (gr_line (start 33.02 27.94) (end 76.2 27.94) (layer Edge.Cuts) (width 0.15))
 (segment (start 114.3 91.44) (end 129.54 91.44) (width 2) (layer B.Cu) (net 2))
 (segment (start 114.3 30.48) (end 114.3 91.44) (width 2) (layer B.Cu) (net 2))
 (segment (start 114.3 36.83) (end 114.3 54.61) (width 2) (layer F.Cu) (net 14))
 (segment (start 114.3 29.21) (end 114.3 36.83) (width 2) (layer F.Cu) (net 14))
 (segment (start 114.3 54.61) (end 114.3 91.44) (width 2) (layer F.Cu) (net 14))
 (segment (start 114.3 91.44) (end 129.54 91.44) (width 2) (layer F.Cu) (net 14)))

